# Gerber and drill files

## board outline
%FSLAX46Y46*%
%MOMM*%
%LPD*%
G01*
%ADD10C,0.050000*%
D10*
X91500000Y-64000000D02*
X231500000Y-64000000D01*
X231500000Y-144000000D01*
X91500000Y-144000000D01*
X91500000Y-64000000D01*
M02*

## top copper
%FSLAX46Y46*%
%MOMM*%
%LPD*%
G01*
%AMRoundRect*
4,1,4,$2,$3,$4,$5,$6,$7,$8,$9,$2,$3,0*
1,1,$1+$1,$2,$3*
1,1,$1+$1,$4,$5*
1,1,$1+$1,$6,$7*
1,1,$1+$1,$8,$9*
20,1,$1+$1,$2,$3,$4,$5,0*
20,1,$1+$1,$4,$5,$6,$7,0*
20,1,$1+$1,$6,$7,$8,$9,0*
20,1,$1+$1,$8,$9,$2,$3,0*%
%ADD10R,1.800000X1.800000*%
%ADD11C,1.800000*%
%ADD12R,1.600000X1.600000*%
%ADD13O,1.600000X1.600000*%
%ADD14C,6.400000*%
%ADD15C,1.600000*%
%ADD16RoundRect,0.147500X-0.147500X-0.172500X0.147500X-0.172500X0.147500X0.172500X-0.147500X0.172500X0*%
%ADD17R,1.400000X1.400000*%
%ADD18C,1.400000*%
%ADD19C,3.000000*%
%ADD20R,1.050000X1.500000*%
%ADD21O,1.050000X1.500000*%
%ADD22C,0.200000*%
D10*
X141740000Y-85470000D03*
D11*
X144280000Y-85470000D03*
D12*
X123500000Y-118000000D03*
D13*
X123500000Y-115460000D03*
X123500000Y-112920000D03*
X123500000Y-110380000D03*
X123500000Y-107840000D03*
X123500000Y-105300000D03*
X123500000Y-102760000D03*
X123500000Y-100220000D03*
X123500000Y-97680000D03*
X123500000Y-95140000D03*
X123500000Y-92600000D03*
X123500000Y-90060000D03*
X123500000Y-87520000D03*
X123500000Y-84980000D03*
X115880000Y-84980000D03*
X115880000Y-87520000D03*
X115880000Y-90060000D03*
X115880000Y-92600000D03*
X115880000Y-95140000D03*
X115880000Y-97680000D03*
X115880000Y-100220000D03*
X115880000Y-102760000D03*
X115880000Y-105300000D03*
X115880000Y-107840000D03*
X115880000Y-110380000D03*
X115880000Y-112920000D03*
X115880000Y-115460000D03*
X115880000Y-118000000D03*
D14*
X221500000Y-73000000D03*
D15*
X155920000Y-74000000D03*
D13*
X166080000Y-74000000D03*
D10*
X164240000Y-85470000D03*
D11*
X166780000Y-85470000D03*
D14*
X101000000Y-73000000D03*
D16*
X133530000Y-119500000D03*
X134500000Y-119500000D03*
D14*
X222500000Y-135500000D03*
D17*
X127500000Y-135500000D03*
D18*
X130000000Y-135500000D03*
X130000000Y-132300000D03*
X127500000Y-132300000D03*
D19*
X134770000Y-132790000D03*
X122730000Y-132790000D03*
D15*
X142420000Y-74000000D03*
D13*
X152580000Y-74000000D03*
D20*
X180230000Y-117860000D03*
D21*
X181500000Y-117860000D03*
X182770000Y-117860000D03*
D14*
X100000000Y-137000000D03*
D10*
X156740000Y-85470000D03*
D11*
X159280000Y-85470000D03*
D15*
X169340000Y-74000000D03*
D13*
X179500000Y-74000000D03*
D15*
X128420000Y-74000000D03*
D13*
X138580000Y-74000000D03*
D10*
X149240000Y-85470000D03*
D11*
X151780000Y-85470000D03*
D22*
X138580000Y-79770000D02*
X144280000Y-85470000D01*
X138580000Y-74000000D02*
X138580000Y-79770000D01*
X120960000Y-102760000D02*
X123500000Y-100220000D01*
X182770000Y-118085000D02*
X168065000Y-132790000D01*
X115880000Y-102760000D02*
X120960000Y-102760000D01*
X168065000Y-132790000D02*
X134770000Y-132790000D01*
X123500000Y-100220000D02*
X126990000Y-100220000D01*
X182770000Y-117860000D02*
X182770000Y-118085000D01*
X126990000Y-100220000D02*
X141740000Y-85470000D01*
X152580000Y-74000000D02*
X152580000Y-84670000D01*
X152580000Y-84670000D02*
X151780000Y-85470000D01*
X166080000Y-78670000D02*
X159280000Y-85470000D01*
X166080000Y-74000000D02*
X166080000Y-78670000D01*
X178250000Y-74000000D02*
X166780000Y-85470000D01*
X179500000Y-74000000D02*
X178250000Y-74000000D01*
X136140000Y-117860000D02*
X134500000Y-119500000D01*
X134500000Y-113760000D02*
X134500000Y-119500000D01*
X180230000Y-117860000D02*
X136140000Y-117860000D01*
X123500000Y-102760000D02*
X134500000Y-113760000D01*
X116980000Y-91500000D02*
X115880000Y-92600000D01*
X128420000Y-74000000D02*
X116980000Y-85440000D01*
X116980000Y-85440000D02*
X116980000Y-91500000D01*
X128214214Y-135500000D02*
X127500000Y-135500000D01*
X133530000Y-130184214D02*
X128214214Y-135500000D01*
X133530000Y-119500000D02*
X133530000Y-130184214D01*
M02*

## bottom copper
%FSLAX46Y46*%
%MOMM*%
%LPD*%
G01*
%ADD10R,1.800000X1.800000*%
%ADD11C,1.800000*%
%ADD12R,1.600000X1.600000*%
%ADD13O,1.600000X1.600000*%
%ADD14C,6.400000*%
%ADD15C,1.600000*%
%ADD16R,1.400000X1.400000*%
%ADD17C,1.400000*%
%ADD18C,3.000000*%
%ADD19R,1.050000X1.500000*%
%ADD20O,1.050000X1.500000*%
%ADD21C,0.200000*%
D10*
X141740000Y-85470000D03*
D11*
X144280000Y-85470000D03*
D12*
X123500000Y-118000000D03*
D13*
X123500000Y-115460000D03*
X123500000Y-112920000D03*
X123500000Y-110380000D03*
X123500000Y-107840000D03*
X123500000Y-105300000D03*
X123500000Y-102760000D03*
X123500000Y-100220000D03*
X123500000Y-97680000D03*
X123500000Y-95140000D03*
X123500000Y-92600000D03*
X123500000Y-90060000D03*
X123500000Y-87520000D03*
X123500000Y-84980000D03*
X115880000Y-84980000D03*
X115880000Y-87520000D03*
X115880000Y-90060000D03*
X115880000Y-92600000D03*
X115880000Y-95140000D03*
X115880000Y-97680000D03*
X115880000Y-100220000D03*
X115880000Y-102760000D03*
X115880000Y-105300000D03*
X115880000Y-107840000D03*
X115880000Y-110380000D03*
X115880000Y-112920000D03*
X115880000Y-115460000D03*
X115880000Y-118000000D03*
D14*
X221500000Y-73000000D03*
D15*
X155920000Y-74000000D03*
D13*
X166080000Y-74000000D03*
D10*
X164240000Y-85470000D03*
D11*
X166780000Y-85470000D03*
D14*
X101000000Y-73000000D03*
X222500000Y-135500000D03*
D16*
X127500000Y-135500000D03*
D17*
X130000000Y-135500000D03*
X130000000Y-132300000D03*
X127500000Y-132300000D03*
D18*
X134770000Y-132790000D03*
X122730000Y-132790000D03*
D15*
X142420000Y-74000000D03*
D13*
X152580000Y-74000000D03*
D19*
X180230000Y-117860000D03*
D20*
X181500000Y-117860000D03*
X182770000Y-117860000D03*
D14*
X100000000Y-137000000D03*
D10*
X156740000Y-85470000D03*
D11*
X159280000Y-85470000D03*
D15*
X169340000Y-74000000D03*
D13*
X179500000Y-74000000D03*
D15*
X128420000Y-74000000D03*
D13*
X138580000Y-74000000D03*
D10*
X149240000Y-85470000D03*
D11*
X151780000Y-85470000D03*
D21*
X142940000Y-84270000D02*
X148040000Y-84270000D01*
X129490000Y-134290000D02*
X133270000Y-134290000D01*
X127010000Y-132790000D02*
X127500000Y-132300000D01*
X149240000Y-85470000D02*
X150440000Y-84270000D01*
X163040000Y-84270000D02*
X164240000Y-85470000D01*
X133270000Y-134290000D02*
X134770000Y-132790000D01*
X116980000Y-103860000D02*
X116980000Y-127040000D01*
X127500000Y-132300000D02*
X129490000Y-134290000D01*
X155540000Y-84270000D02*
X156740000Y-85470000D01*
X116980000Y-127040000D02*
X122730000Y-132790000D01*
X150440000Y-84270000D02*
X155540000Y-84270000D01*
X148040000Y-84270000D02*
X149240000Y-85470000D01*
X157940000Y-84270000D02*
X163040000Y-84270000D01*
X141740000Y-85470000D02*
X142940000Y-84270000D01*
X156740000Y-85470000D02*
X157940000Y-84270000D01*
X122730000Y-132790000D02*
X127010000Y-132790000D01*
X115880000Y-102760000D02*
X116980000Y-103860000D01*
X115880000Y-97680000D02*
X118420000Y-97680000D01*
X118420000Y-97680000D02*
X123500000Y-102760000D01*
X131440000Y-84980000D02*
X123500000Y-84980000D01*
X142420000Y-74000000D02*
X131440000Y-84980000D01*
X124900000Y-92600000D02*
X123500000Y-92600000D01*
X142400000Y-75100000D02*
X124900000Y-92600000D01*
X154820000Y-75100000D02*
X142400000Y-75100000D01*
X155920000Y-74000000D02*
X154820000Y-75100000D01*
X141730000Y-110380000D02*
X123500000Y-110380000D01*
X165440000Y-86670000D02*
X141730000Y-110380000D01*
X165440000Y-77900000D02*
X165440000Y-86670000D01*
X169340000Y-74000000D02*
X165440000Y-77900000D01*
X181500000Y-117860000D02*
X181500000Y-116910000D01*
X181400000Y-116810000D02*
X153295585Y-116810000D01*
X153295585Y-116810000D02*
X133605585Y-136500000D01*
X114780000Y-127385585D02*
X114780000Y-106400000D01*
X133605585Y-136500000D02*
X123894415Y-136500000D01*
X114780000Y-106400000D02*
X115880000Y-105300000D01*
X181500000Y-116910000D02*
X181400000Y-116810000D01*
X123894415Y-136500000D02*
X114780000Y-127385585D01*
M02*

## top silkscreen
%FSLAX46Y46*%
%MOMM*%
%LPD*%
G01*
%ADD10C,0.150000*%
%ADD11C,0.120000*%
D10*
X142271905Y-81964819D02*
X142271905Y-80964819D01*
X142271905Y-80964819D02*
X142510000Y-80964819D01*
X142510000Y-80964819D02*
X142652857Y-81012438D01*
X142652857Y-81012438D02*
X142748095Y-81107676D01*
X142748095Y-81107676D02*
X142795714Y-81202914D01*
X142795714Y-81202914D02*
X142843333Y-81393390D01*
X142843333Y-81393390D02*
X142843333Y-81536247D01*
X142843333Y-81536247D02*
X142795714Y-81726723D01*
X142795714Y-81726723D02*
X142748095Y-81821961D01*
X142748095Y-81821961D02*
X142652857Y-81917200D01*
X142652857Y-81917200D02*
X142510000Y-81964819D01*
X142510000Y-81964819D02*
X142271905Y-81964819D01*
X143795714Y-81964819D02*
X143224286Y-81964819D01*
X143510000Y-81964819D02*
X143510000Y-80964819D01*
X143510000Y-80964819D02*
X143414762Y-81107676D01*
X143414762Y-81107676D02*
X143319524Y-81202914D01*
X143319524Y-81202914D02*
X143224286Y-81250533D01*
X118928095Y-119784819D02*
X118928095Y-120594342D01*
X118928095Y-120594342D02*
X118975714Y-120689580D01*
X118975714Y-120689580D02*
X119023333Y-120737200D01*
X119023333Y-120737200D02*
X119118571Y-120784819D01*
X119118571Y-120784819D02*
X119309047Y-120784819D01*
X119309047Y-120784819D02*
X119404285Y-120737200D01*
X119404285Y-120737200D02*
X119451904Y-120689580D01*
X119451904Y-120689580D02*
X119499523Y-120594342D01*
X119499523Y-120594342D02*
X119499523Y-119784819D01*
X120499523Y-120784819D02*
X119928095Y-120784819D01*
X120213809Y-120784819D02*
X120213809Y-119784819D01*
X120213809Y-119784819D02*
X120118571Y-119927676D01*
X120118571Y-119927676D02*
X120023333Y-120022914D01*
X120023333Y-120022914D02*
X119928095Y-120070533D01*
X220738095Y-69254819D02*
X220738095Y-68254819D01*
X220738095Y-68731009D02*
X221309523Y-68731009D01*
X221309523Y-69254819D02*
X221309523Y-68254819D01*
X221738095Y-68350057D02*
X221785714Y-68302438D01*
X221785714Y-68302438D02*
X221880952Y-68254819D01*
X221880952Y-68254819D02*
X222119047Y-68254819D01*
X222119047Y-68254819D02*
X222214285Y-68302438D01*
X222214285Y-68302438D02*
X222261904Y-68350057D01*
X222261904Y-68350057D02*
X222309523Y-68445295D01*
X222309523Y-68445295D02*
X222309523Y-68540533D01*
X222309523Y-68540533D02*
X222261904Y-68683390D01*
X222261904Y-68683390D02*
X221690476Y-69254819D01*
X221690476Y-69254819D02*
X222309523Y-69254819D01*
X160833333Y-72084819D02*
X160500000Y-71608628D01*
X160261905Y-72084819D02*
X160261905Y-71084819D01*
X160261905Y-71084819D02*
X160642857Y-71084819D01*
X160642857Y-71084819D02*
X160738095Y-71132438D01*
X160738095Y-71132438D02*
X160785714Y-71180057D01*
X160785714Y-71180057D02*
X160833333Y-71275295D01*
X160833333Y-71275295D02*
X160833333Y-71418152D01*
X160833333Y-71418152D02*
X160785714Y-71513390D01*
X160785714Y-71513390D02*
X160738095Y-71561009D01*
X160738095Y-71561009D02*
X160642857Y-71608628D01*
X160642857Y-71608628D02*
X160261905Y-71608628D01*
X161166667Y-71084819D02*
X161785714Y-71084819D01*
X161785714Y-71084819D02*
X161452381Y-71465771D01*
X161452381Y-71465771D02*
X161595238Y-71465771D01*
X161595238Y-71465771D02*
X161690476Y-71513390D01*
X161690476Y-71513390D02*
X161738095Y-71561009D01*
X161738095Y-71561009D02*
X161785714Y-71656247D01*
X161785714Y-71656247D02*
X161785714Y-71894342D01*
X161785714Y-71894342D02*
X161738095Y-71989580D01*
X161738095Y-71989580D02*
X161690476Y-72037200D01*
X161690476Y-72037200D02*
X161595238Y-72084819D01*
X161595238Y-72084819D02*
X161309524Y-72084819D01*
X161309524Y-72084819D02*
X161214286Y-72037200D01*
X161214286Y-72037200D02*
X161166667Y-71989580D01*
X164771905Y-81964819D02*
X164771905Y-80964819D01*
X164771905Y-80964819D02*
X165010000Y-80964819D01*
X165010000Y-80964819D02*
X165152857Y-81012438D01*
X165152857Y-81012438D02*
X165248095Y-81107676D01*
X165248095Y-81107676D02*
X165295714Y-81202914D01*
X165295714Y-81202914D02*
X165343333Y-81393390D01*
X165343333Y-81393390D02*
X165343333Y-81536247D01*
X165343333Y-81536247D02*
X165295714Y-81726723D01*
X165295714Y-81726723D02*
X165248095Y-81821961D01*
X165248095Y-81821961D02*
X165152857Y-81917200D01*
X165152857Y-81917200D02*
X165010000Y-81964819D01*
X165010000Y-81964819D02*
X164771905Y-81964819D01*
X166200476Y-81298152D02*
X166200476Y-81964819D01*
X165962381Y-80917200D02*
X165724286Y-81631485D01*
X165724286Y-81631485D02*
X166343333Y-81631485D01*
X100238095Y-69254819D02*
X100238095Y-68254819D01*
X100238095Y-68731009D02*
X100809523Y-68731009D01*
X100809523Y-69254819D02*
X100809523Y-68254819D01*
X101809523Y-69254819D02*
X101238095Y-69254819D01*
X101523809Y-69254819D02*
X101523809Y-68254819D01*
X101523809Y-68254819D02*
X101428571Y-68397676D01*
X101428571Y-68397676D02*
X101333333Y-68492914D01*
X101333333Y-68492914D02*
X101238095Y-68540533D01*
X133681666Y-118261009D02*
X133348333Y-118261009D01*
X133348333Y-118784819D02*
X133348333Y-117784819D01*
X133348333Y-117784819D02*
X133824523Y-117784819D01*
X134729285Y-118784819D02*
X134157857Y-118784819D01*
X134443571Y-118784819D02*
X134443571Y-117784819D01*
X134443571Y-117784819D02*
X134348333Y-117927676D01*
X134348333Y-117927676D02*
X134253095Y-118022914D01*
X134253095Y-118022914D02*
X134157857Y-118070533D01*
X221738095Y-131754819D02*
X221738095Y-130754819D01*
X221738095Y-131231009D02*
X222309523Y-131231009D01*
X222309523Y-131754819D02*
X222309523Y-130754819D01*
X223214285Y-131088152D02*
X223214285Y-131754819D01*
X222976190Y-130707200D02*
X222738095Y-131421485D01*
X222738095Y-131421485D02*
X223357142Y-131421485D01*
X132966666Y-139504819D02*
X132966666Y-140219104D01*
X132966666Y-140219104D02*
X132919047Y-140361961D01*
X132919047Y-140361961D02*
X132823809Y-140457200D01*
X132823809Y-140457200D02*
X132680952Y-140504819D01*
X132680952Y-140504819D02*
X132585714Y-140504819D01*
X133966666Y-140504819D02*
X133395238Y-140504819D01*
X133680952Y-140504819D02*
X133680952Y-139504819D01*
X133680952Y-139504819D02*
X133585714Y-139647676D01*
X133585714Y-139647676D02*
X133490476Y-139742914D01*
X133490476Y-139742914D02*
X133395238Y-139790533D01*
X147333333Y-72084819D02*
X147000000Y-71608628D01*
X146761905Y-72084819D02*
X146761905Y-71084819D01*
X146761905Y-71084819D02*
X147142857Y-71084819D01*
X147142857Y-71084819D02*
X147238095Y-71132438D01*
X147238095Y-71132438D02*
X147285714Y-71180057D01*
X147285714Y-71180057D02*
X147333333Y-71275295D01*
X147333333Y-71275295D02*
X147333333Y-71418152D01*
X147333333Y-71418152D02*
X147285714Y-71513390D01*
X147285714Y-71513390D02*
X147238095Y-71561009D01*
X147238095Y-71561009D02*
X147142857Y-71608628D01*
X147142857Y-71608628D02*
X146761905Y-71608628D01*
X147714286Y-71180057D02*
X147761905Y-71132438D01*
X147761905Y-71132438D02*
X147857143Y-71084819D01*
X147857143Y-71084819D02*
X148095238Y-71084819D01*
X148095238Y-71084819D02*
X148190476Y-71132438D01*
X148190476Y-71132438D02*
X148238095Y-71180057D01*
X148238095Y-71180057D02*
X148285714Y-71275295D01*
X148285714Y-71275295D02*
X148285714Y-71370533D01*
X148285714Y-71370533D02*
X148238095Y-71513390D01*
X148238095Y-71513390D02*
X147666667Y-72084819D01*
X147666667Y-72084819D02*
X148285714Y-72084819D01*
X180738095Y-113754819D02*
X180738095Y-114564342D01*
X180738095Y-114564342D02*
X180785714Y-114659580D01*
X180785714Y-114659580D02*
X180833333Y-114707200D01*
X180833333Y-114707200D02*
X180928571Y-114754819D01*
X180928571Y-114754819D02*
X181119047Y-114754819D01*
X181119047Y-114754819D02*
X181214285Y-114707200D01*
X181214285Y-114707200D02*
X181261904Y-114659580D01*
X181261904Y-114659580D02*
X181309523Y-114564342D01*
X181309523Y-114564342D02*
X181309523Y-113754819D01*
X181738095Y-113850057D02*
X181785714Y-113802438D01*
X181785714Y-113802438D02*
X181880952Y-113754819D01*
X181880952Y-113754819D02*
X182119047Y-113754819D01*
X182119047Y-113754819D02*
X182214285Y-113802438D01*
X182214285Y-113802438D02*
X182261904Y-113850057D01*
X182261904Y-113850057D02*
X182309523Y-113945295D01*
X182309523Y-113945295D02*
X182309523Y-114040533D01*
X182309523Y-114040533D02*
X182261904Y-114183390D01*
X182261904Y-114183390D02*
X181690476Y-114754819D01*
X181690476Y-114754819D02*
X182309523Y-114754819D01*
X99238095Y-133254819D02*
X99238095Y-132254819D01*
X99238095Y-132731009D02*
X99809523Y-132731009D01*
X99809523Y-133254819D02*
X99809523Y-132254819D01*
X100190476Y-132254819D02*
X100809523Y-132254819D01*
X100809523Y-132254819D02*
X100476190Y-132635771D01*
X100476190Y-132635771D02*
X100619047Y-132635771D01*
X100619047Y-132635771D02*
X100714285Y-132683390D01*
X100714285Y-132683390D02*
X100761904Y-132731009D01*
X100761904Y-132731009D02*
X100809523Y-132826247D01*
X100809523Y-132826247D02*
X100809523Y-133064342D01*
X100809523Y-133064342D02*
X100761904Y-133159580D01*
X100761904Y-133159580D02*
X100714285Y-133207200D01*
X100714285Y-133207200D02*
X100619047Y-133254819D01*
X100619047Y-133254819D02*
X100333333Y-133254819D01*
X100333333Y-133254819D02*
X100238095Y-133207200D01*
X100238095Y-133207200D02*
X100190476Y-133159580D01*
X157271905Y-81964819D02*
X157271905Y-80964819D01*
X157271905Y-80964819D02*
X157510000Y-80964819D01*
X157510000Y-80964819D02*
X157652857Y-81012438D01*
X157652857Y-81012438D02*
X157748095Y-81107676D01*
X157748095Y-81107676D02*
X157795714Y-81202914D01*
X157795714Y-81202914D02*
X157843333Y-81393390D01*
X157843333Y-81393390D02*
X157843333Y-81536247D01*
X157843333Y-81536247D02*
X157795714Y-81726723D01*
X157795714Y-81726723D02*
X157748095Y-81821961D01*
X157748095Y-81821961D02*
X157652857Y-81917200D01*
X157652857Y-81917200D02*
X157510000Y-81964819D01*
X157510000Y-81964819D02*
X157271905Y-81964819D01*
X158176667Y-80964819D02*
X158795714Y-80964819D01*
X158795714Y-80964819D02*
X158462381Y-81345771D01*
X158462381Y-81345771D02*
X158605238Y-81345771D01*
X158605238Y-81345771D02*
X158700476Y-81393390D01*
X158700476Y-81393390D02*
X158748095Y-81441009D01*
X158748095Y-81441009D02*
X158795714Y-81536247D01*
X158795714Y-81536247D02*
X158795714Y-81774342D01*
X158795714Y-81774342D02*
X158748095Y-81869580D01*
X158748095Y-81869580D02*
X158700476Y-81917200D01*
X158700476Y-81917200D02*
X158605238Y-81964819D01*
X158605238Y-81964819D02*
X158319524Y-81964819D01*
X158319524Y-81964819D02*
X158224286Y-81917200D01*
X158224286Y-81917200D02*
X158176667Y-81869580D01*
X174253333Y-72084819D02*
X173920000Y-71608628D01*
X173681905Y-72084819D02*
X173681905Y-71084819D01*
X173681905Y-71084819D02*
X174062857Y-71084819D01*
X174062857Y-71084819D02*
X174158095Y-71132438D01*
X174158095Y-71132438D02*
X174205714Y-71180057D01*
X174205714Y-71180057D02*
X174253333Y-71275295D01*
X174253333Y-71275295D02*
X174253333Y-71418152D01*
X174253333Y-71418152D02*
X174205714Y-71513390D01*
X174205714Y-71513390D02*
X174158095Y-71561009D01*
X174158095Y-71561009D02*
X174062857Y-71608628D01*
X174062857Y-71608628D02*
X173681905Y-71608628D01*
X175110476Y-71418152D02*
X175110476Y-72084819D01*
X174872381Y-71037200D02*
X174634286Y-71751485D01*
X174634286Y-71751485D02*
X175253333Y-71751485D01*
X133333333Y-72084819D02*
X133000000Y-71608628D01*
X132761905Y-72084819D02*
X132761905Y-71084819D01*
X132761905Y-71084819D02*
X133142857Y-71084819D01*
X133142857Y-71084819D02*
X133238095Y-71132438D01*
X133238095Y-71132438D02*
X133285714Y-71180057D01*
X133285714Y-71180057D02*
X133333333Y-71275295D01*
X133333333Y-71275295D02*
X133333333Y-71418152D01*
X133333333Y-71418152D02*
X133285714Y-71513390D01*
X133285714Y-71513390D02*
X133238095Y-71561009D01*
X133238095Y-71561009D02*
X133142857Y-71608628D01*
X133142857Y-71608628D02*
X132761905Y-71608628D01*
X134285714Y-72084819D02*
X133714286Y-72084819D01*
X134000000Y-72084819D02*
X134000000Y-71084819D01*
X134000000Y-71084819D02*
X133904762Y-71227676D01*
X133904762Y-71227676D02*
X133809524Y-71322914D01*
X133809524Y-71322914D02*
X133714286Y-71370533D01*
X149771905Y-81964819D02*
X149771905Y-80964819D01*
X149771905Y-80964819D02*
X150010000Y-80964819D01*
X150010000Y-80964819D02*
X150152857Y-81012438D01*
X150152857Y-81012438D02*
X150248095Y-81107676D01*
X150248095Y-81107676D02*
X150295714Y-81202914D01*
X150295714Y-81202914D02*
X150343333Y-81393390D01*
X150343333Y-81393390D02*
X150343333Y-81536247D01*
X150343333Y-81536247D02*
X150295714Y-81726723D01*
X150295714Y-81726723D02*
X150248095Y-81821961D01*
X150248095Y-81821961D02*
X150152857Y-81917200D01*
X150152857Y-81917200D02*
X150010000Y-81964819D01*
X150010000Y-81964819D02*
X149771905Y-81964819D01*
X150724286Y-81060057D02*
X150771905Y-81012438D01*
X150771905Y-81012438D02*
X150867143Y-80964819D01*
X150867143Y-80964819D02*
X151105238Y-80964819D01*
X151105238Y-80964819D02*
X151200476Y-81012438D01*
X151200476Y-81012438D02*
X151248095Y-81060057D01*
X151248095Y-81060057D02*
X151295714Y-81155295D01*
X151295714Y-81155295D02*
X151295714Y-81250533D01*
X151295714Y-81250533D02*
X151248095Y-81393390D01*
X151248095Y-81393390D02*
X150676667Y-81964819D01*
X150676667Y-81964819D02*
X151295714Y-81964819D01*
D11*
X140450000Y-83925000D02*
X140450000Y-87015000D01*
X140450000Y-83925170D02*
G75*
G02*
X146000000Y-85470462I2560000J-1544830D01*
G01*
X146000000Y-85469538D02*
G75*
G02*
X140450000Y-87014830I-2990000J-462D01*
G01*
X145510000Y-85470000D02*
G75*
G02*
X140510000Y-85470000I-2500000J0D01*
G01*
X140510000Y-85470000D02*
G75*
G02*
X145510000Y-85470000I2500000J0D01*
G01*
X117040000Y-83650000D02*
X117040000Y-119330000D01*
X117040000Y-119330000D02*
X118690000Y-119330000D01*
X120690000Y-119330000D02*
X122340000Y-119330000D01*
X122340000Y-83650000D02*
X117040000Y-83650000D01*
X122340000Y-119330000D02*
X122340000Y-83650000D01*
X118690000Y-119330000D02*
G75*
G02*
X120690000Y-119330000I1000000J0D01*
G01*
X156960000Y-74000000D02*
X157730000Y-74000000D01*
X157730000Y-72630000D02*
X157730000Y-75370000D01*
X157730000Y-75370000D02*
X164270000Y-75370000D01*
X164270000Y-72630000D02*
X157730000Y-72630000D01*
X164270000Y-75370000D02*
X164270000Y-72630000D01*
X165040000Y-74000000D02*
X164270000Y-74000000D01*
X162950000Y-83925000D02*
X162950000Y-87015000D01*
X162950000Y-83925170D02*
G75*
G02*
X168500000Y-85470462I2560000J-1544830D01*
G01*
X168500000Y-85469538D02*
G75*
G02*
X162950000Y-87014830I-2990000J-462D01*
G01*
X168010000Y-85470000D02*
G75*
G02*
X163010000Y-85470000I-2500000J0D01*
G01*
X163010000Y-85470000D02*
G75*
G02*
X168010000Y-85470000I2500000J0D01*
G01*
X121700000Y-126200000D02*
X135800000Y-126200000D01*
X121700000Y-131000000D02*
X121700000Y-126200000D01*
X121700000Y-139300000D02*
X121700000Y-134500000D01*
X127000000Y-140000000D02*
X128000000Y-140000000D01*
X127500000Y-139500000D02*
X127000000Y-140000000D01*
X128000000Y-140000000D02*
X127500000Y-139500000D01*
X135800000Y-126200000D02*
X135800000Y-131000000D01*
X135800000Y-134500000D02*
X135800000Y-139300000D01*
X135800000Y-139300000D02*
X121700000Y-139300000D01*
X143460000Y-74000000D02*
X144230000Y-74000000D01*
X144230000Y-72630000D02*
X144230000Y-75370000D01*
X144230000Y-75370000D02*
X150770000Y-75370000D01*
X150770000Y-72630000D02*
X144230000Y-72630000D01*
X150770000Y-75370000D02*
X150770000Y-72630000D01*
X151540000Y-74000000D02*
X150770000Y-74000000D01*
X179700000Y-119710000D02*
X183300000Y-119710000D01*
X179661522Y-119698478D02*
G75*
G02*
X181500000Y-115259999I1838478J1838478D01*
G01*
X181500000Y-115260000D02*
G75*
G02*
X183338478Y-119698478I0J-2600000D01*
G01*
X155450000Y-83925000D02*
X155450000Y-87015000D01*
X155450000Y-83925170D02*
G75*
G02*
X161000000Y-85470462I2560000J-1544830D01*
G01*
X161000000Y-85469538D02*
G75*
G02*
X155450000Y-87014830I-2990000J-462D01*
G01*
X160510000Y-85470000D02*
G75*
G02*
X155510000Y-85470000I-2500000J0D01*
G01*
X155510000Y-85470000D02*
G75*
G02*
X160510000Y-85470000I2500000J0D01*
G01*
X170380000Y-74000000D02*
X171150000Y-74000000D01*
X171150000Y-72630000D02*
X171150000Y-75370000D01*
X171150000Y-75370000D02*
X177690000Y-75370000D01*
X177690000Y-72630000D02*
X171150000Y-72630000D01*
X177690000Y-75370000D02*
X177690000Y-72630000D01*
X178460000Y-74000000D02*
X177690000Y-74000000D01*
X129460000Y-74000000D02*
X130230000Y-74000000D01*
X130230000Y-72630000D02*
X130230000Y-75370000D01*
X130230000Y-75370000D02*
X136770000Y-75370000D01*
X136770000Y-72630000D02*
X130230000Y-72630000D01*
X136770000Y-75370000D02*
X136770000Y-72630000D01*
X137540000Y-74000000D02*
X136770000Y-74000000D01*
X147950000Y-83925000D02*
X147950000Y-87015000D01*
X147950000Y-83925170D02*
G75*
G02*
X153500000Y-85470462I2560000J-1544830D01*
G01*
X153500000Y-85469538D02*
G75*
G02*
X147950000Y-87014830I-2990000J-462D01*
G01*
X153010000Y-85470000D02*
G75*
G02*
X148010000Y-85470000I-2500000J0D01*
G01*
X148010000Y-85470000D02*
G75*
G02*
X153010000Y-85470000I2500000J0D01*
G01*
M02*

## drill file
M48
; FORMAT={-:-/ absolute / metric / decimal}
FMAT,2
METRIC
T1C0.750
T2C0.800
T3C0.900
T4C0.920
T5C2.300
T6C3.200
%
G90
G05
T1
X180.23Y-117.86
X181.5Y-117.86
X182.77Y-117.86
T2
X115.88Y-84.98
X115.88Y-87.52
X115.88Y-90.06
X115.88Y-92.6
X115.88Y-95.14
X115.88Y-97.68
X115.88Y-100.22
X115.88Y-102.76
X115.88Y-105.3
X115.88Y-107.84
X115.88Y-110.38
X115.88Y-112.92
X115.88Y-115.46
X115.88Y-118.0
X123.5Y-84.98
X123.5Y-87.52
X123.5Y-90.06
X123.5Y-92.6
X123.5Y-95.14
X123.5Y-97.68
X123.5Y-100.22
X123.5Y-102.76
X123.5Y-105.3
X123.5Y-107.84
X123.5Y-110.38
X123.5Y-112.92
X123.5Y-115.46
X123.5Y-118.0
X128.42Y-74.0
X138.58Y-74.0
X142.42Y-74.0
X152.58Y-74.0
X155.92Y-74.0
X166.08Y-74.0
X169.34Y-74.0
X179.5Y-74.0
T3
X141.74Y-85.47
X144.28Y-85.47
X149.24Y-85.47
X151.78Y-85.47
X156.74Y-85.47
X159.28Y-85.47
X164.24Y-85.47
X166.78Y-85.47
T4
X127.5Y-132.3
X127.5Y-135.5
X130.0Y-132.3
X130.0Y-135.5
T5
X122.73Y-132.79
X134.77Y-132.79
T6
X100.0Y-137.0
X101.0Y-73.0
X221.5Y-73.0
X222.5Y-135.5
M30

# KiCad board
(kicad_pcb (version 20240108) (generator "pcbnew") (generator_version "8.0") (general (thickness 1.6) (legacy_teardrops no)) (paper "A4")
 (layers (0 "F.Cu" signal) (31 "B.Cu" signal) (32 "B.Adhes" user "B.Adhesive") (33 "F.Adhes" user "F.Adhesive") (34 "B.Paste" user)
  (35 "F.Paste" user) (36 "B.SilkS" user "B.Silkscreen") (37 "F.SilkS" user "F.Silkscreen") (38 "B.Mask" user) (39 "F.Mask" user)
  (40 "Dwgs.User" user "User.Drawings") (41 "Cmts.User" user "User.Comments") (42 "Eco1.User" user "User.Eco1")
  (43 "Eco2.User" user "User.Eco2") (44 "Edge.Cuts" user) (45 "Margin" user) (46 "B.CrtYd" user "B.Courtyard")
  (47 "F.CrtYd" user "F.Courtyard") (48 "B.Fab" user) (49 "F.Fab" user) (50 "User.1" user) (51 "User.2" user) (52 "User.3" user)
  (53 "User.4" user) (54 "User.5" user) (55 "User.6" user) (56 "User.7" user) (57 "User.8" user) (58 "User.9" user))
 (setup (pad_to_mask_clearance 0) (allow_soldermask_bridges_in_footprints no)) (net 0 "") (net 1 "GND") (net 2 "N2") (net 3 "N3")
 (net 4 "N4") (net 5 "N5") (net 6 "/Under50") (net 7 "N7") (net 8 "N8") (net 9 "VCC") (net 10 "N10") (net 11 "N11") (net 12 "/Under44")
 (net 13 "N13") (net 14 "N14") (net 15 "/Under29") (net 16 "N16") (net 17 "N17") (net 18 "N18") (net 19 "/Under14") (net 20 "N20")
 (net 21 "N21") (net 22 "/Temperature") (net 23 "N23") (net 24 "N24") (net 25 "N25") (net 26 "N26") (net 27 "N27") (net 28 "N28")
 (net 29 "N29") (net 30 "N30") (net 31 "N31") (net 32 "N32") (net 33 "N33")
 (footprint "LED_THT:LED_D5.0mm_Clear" (layer "F.Cu") (at 141.74 85.47)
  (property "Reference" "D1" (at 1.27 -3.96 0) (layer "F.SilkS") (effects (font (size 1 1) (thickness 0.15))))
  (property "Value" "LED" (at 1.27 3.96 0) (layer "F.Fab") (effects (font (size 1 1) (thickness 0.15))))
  (fp_line (start -1.29 -1.545) (end -1.29 1.545) (stroke (width 0.12) (type solid)) (layer "F.SilkS"))
  (fp_arc (start -1.29 -1.54483) (mid 2.072002 -2.880433) (end 4.26 0.000462) (stroke (width 0.12) (type solid)) (layer "F.SilkS"))
  (fp_arc (start 4.26 -0.000462) (mid 2.072002 2.880433) (end -1.29 1.54483) (stroke (width 0.12) (type solid)) (layer "F.SilkS"))
  (fp_circle (center 1.27 0) (end 3.77 0) (stroke (width 0.12) (type solid)) (fill none) (layer "F.SilkS"))
  (pad "1" thru_hole rect (at 0 0) (size 1.8 1.8) (drill 0.9) (layers "*.Cu" "*.Mask") (remove_unused_layers no) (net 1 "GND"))
  (pad "2" thru_hole circle (at 2.54 0) (size 1.8 1.8) (drill 0.9) (layers "*.Cu" "*.Mask") (remove_unused_layers no) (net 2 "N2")))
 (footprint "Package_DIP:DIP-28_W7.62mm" (layer "F.Cu") (at 123.5 118 180)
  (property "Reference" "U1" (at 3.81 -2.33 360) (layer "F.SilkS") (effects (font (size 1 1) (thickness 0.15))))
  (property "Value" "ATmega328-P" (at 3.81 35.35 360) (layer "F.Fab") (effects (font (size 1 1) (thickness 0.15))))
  (fp_line (start 6.46 34.35) (end 6.46 -1.33) (stroke (width 0.12) (type solid)) (layer "F.SilkS"))
  (fp_line (start 6.46 -1.33) (end 4.81 -1.33) (stroke (width 0.12) (type solid)) (layer "F.SilkS"))
  (fp_line (start 2.81 -1.33) (end 1.16 -1.33) (stroke (width 0.12) (type solid)) (layer "F.SilkS"))
  (fp_line (start 1.16 34.35) (end 6.46 34.35) (stroke (width 0.12) (type solid)) (layer "F.SilkS"))
  (fp_line (start 1.16 -1.33) (end 1.16 34.35) (stroke (width 0.12) (type solid)) (layer "F.SilkS"))
  (fp_arc (start 4.81 -1.33) (mid 3.81 -0.33) (end 2.81 -1.33) (stroke (width 0.12) (type solid)) (layer "F.SilkS"))
  (pad "1" thru_hole rect (at 0 0 180) (size 1.6 1.6) (drill 0.8) (layers "*.Cu" "*.Mask") (remove_unused_layers no) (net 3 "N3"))
  (pad "2" thru_hole oval (at 0 2.54 180) (size 1.6 1.6) (drill 0.8) (layers "*.Cu" "*.Mask") (remove_unused_layers no) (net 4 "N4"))
  (pad "3" thru_hole oval (at 0 5.08 180) (size 1.6 1.6) (drill 0.8) (layers "*.Cu" "*.Mask") (remove_unused_layers no) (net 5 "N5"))
  (pad "4" thru_hole oval (at 0 7.62 180) (size 1.6 1.6) (drill 0.8) (layers "*.Cu" "*.Mask") (remove_unused_layers no) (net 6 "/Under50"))
  (pad "5" thru_hole oval (at 0 10.16 180) (size 1.6 1.6) (drill 0.8) (layers "*.Cu" "*.Mask") (remove_unused_layers no) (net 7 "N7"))
  (pad "6" thru_hole oval (at 0 12.7 180) (size 1.6 1.6) (drill 0.8) (layers "*.Cu" "*.Mask") (remove_unused_layers no) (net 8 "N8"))
  (pad "7" thru_hole oval (at 0 15.24 180) (size 1.6 1.6) (drill 0.8) (layers "*.Cu" "*.Mask") (remove_unused_layers no) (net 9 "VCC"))
  (pad "8" thru_hole oval (at 0 17.78 180) (size 1.6 1.6) (drill 0.8) (layers "*.Cu" "*.Mask") (remove_unused_layers no) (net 1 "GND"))
  (pad "9" thru_hole oval (at 0 20.32 180) (size 1.6 1.6) (drill 0.8) (layers "*.Cu" "*.Mask") (remove_unused_layers no) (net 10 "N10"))
  (pad "10" thru_hole oval (at 0 22.86 180) (size 1.6 1.6) (drill 0.8) (layers "*.Cu" "*.Mask") (remove_unused_layers no) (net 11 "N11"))
  (pad "11" thru_hole oval (at 0 25.4 180) (size 1.6 1.6) (drill 0.8) (layers "*.Cu" "*.Mask") (remove_unused_layers no) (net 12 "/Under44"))
  (pad "12" thru_hole oval (at 0 27.94 180) (size 1.6 1.6) (drill 0.8) (layers "*.Cu" "*.Mask") (remove_unused_layers no) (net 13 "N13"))
  (pad "13" thru_hole oval (at 0 30.48 180) (size 1.6 1.6) (drill 0.8) (layers "*.Cu" "*.Mask") (remove_unused_layers no) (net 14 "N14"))
  (pad "14" thru_hole oval (at 0 33.02 180) (size 1.6 1.6) (drill 0.8) (layers "*.Cu" "*.Mask") (remove_unused_layers no)
   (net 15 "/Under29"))
  (pad "15" thru_hole oval (at 7.62 33.02 180) (size 1.6 1.6) (drill 0.8) (layers "*.Cu" "*.Mask") (remove_unused_layers no) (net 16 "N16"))
  (pad "16" thru_hole oval (at 7.62 30.48 180) (size 1.6 1.6) (drill 0.8) (layers "*.Cu" "*.Mask") (remove_unused_layers no) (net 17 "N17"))
  (pad "17" thru_hole oval (at 7.62 27.94 180) (size 1.6 1.6) (drill 0.8) (layers "*.Cu" "*.Mask") (remove_unused_layers no) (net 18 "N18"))
  (pad "18" thru_hole oval (at 7.62 25.4 180) (size 1.6 1.6) (drill 0.8) (layers "*.Cu" "*.Mask") (remove_unused_layers no)
   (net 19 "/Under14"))
  (pad "19" thru_hole oval (at 7.62 22.86 180) (size 1.6 1.6) (drill 0.8) (layers "*.Cu" "*.Mask") (remove_unused_layers no) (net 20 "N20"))
  (pad "20" thru_hole oval (at 7.62 20.32 180) (size 1.6 1.6) (drill 0.8) (layers "*.Cu" "*.Mask") (remove_unused_layers no) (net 9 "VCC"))
  (pad "21" thru_hole oval (at 7.62 17.78 180) (size 1.6 1.6) (drill 0.8) (layers "*.Cu" "*.Mask") (remove_unused_layers no) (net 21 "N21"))
  (pad "22" thru_hole oval (at 7.62 15.24 180) (size 1.6 1.6) (drill 0.8) (layers "*.Cu" "*.Mask") (remove_unused_layers no) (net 1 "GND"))
  (pad "23" thru_hole oval (at 7.62 12.7 180) (size 1.6 1.6) (drill 0.8) (layers "*.Cu" "*.Mask") (remove_unused_layers no)
   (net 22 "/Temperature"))
  (pad "24" thru_hole oval (at 7.62 10.16 180) (size 1.6 1.6) (drill 0.8) (layers "*.Cu" "*.Mask") (remove_unused_layers no) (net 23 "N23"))
  (pad "25" thru_hole oval (at 7.62 7.62 180) (size 1.6 1.6) (drill 0.8) (layers "*.Cu" "*.Mask") (remove_unused_layers no) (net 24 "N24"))
  (pad "26" thru_hole oval (at 7.62 5.08 180) (size 1.6 1.6) (drill 0.8) (layers "*.Cu" "*.Mask") (remove_unused_layers no) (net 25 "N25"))
  (pad "27" thru_hole oval (at 7.62 2.54 180) (size 1.6 1.6) (drill 0.8) (layers "*.Cu" "*.Mask") (remove_unused_layers no) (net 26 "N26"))
  (pad "28" thru_hole oval (at 7.62 0 180) (size 1.6 1.6) (drill 0.8) (layers "*.Cu" "*.Mask") (remove_unused_layers no) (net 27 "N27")))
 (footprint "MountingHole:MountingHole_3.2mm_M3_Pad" (layer "F.Cu") (at 221.5 73)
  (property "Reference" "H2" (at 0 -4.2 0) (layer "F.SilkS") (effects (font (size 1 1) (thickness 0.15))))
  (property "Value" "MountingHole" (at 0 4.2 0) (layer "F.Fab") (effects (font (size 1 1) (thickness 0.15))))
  (pad "1" thru_hole circle (at 0 0) (size 6.4 6.4) (drill 3.2) (layers "*.Cu" "*.Mask") (remove_unused_layers no)))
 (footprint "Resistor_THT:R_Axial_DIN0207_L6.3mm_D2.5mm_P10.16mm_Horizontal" (layer "F.Cu") (at 155.92 74)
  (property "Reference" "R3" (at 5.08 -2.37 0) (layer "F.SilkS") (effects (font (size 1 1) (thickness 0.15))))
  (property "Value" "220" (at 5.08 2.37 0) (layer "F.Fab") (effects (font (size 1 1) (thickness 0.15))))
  (fp_line (start 1.04 0) (end 1.81 0) (stroke (width 0.12) (type solid)) (layer "F.SilkS"))
  (fp_line (start 1.81 -1.37) (end 1.81 1.37) (stroke (width 0.12) (type solid)) (layer "F.SilkS"))
  (fp_line (start 1.81 1.37) (end 8.35 1.37) (stroke (width 0.12) (type solid)) (layer "F.SilkS"))
  (fp_line (start 8.35 -1.37) (end 1.81 -1.37) (stroke (width 0.12) (type solid)) (layer "F.SilkS"))
  (fp_line (start 8.35 1.37) (end 8.35 -1.37) (stroke (width 0.12) (type solid)) (layer "F.SilkS"))
  (fp_line (start 9.12 0) (end 8.35 0) (stroke (width 0.12) (type solid)) (layer "F.SilkS"))
  (pad "1" thru_hole circle (at 0 0) (size 1.6 1.6) (drill 0.8) (layers "*.Cu" "*.Mask") (remove_unused_layers no) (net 12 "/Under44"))
  (pad "2" thru_hole oval (at 10.16 0) (size 1.6 1.6) (drill 0.8) (layers "*.Cu" "*.Mask") (remove_unused_layers no) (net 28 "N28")))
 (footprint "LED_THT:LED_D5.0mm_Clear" (layer "F.Cu") (at 164.24 85.47)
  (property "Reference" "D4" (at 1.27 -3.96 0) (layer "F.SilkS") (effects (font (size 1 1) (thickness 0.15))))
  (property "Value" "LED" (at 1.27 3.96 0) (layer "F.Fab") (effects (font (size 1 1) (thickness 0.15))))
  (fp_line (start -1.29 -1.545) (end -1.29 1.545) (stroke (width 0.12) (type solid)) (layer "F.SilkS"))
  (fp_arc (start -1.29 -1.54483) (mid 2.072002 -2.880433) (end 4.26 0.000462) (stroke (width 0.12) (type solid)) (layer "F.SilkS"))
  (fp_arc (start 4.26 -0.000462) (mid 2.072002 2.880433) (end -1.29 1.54483) (stroke (width 0.12) (type solid)) (layer "F.SilkS"))
  (fp_circle (center 1.27 0) (end 3.77 0) (stroke (width 0.12) (type solid)) (fill none) (layer "F.SilkS"))
  (pad "1" thru_hole rect (at 0 0) (size 1.8 1.8) (drill 0.9) (layers "*.Cu" "*.Mask") (remove_unused_layers no) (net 1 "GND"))
  (pad "2" thru_hole circle (at 2.54 0) (size 1.8 1.8) (drill 0.9) (layers "*.Cu" "*.Mask") (remove_unused_layers no) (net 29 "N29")))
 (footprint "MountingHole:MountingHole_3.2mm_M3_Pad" (layer "F.Cu") (at 101 73)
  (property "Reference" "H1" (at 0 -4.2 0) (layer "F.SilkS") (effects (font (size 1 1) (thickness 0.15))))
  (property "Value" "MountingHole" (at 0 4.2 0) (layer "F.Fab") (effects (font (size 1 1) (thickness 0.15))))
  (pad "1" thru_hole circle (at 0 0) (size 6.4 6.4) (drill 3.2) (layers "*.Cu" "*.Mask") (remove_unused_layers no)))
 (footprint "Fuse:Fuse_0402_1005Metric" (layer "F.Cu") (at 134.015 119.5)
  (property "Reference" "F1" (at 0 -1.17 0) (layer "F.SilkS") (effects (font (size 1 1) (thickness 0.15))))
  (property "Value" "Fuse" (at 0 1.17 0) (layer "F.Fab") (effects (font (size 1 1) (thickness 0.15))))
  (pad "1" smd roundrect (at -0.485 0) (size 0.59 0.64) (layers "F.Cu" "F.Paste" "F.Mask") (roundrect_rratio 0.25) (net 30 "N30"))
  (pad "2" smd roundrect (at 0.485 0) (size 0.59 0.64) (layers "F.Cu" "F.Paste" "F.Mask") (roundrect_rratio 0.25) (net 9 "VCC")))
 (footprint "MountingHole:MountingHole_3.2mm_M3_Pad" (layer "F.Cu") (at 222.5 135.5)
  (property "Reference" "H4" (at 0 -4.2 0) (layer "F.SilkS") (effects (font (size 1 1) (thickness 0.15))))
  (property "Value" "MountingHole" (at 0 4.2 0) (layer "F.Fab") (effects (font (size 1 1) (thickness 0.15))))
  (pad "1" thru_hole circle (at 0 0) (size 6.4 6.4) (drill 3.2) (layers "*.Cu" "*.Mask") (remove_unused_layers no)))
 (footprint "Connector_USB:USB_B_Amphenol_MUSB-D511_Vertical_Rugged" (layer "F.Cu") (at 127.5 135.5 180)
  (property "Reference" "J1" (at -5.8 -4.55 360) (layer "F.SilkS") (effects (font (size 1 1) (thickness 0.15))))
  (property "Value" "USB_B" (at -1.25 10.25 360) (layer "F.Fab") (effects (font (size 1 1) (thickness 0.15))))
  (fp_line (start 5.8 9.3) (end -8.3 9.3) (stroke (width 0.12) (type solid)) (layer "F.SilkS"))
  (fp_line (start 5.8 4.5) (end 5.8 9.3) (stroke (width 0.12) (type solid)) (layer "F.SilkS"))
  (fp_line (start 5.8 -3.8) (end 5.8 1) (stroke (width 0.12) (type solid)) (layer "F.SilkS"))
  (fp_line (start 0.5 -4.5) (end -0.5 -4.5) (stroke (width 0.12) (type solid)) (layer "F.SilkS"))
  (fp_line (start 0 -4) (end 0.5 -4.5) (stroke (width 0.12) (type solid)) (layer "F.SilkS"))
  (fp_line (start -0.5 -4.5) (end 0 -4) (stroke (width 0.12) (type solid)) (layer "F.SilkS"))
  (fp_line (start -8.3 9.3) (end -8.3 4.5) (stroke (width 0.12) (type solid)) (layer "F.SilkS"))
  (fp_line (start -8.3 1) (end -8.3 -3.8) (stroke (width 0.12) (type solid)) (layer "F.SilkS"))
  (fp_line (start -8.3 -3.8) (end 5.8 -3.8) (stroke (width 0.12) (type solid)) (layer "F.SilkS"))
  (pad "1" thru_hole rect (at 0 0 180) (size 1.4 1.4) (drill 0.92) (layers "*.Cu" "*.Mask") (remove_unused_layers no) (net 30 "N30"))
  (pad "2" thru_hole circle (at -2.5 0 180) (size 1.4 1.4) (drill 0.92) (layers "*.Cu" "*.Mask") (remove_unused_layers no) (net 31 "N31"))
  (pad "3" thru_hole circle (at -2.5 3.2 180) (size 1.4 1.4) (drill 0.92) (layers "*.Cu" "*.Mask") (remove_unused_layers no) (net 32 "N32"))
  (pad "4" thru_hole circle (at 0 3.2 180) (size 1.4 1.4) (drill 0.92) (layers "*.Cu" "*.Mask") (remove_unused_layers no) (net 1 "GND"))
  (pad "5" thru_hole circle (at -7.27 2.71 180) (size 3 3) (drill 2.3) (layers "*.Cu" "*.Mask") (remove_unused_layers no) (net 1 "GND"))
  (pad "5" thru_hole circle (at 4.77 2.71 180) (size 3 3) (drill 2.3) (layers "*.Cu" "*.Mask") (remove_unused_layers no) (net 1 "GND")))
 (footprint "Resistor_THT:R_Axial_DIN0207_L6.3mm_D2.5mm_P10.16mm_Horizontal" (layer "F.Cu") (at 142.42 74)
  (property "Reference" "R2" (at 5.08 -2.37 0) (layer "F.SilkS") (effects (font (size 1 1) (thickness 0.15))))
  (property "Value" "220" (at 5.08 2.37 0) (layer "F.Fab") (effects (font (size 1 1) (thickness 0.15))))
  (fp_line (start 1.04 0) (end 1.81 0) (stroke (width 0.12) (type solid)) (layer "F.SilkS"))
  (fp_line (start 1.81 -1.37) (end 1.81 1.37) (stroke (width 0.12) (type solid)) (layer "F.SilkS"))
  (fp_line (start 1.81 1.37) (end 8.35 1.37) (stroke (width 0.12) (type solid)) (layer "F.SilkS"))
  (fp_line (start 8.35 -1.37) (end 1.81 -1.37) (stroke (width 0.12) (type solid)) (layer "F.SilkS"))
  (fp_line (start 8.35 1.37) (end 8.35 -1.37) (stroke (width 0.12) (type solid)) (layer "F.SilkS"))
  (fp_line (start 9.12 0) (end 8.35 0) (stroke (width 0.12) (type solid)) (layer "F.SilkS"))
  (pad "1" thru_hole circle (at 0 0) (size 1.6 1.6) (drill 0.8) (layers "*.Cu" "*.Mask") (remove_unused_layers no) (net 15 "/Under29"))
  (pad "2" thru_hole oval (at 10.16 0) (size 1.6 1.6) (drill 0.8) (layers "*.Cu" "*.Mask") (remove_unused_layers no) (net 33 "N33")))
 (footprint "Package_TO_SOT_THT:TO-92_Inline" (layer "F.Cu") (at 180.23 117.86)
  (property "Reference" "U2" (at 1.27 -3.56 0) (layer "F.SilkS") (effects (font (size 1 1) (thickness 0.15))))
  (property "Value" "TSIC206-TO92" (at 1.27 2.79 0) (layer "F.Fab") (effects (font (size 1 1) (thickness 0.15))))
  (fp_line (start -0.53 1.85) (end 3.07 1.85) (stroke (width 0.12) (type solid)) (layer "F.SilkS"))
  (fp_arc (start -0.568478 1.838478) (mid -1.132087 -0.994977) (end 1.27 -2.6) (stroke (width 0.12) (type solid)) (layer "F.SilkS"))
  (fp_arc (start 1.27 -2.6) (mid 3.672087 -0.994977) (end 3.108478 1.838478) (stroke (width 0.12) (type solid)) (layer "F.SilkS"))
  (pad "1" thru_hole rect (at 0 0) (size 1.05 1.5) (drill 0.75) (layers "*.Cu" "*.Mask") (remove_unused_layers no) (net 9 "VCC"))
  (pad "2" thru_hole oval (at 1.27 0) (size 1.05 1.5) (drill 0.75) (layers "*.Cu" "*.Mask") (remove_unused_layers no)
   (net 22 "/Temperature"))
  (pad "3" thru_hole oval (at 2.54 0) (size 1.05 1.5) (drill 0.75) (layers "*.Cu" "*.Mask") (remove_unused_layers no) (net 1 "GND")))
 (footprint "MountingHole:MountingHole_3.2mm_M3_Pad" (layer "F.Cu") (at 100 137)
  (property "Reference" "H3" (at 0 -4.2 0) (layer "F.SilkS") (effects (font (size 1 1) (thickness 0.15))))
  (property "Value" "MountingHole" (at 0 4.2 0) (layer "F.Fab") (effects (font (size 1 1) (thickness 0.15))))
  (pad "1" thru_hole circle (at 0 0) (size 6.4 6.4) (drill 3.2) (layers "*.Cu" "*.Mask") (remove_unused_layers no)))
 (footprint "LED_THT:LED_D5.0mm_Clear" (layer "F.Cu") (at 156.74 85.47)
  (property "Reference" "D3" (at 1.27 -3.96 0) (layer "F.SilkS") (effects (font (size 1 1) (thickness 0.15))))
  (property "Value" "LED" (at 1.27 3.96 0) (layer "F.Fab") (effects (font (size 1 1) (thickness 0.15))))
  (fp_line (start -1.29 -1.545) (end -1.29 1.545) (stroke (width 0.12) (type solid)) (layer "F.SilkS"))
  (fp_arc (start -1.29 -1.54483) (mid 2.072002 -2.880433) (end 4.26 0.000462) (stroke (width 0.12) (type solid)) (layer "F.SilkS"))
  (fp_arc (start 4.26 -0.000462) (mid 2.072002 2.880433) (end -1.29 1.54483) (stroke (width 0.12) (type solid)) (layer "F.SilkS"))
  (fp_circle (center 1.27 0) (end 3.77 0) (stroke (width 0.12) (type solid)) (fill none) (layer "F.SilkS"))
  (pad "1" thru_hole rect (at 0 0) (size 1.8 1.8) (drill 0.9) (layers "*.Cu" "*.Mask") (remove_unused_layers no) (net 1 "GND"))
  (pad "2" thru_hole circle (at 2.54 0) (size 1.8 1.8) (drill 0.9) (layers "*.Cu" "*.Mask") (remove_unused_layers no) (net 28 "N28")))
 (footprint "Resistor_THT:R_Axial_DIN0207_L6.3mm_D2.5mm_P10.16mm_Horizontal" (layer "F.Cu") (at 169.34 74)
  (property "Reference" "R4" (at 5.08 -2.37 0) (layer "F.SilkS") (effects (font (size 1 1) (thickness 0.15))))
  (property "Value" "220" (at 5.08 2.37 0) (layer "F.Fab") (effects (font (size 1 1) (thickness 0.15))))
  (fp_line (start 1.04 0) (end 1.81 0) (stroke (width 0.12) (type solid)) (layer "F.SilkS"))
  (fp_line (start 1.81 -1.37) (end 1.81 1.37) (stroke (width 0.12) (type solid)) (layer "F.SilkS"))
  (fp_line (start 1.81 1.37) (end 8.35 1.37) (stroke (width 0.12) (type solid)) (layer "F.SilkS"))
  (fp_line (start 8.35 -1.37) (end 1.81 -1.37) (stroke (width 0.12) (type solid)) (layer "F.SilkS"))
  (fp_line (start 8.35 1.37) (end 8.35 -1.37) (stroke (width 0.12) (type solid)) (layer "F.SilkS"))
  (fp_line (start 9.12 0) (end 8.35 0) (stroke (width 0.12) (type solid)) (layer "F.SilkS"))
  (pad "1" thru_hole circle (at 0 0) (size 1.6 1.6) (drill 0.8) (layers "*.Cu" "*.Mask") (remove_unused_layers no) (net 6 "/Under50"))
  (pad "2" thru_hole oval (at 10.16 0) (size 1.6 1.6) (drill 0.8) (layers "*.Cu" "*.Mask") (remove_unused_layers no) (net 29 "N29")))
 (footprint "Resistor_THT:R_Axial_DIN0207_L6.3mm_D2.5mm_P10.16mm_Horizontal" (layer "F.Cu") (at 128.42 74)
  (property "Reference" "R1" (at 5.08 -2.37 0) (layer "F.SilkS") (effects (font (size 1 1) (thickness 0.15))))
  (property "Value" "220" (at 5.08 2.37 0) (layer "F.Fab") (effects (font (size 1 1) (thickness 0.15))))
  (fp_line (start 1.04 0) (end 1.81 0) (stroke (width 0.12) (type solid)) (layer "F.SilkS"))
  (fp_line (start 1.81 -1.37) (end 1.81 1.37) (stroke (width 0.12) (type solid)) (layer "F.SilkS"))
  (fp_line (start 1.81 1.37) (end 8.35 1.37) (stroke (width 0.12) (type solid)) (layer "F.SilkS"))
  (fp_line (start 8.35 -1.37) (end 1.81 -1.37) (stroke (width 0.12) (type solid)) (layer "F.SilkS"))
  (fp_line (start 8.35 1.37) (end 8.35 -1.37) (stroke (width 0.12) (type solid)) (layer "F.SilkS"))
  (fp_line (start 9.12 0) (end 8.35 0) (stroke (width 0.12) (type solid)) (layer "F.SilkS"))
  (pad "1" thru_hole circle (at 0 0) (size 1.6 1.6) (drill 0.8) (layers "*.Cu" "*.Mask") (remove_unused_layers no) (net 19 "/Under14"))
  (pad "2" thru_hole oval (at 10.16 0) (size 1.6 1.6) (drill 0.8) (layers "*.Cu" "*.Mask") (remove_unused_layers no) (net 2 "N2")))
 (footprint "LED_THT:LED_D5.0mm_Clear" (layer "F.Cu") (at 149.24 85.47)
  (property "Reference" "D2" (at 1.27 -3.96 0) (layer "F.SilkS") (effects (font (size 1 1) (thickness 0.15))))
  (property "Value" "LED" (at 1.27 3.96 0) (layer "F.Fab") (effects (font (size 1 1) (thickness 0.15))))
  (fp_line (start -1.29 -1.545) (end -1.29 1.545) (stroke (width 0.12) (type solid)) (layer "F.SilkS"))
  (fp_arc (start -1.29 -1.54483) (mid 2.072002 -2.880433) (end 4.26 0.000462) (stroke (width 0.12) (type solid)) (layer "F.SilkS"))
  (fp_arc (start 4.26 -0.000462) (mid 2.072002 2.880433) (end -1.29 1.54483) (stroke (width 0.12) (type solid)) (layer "F.SilkS"))
  (fp_circle (center 1.27 0) (end 3.77 0) (stroke (width 0.12) (type solid)) (fill none) (layer "F.SilkS"))
  (pad "1" thru_hole rect (at 0 0) (size 1.8 1.8) (drill 0.9) (layers "*.Cu" "*.Mask") (remove_unused_layers no) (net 1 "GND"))
  (pad "2" thru_hole circle (at 2.54 0) (size 1.8 1.8) (drill 0.9) (layers "*.Cu" "*.Mask") (remove_unused_layers no) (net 33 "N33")))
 (gr_rect (start 91.5 64) (end 231.5 144) (stroke (width 0.05) (type default)) (fill none) (layer "Edge.Cuts"))
 (segment (start 138.58 79.77) (end 144.28 85.47) (width 0.2) (layer "F.Cu") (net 2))
 (segment (start 138.58 74) (end 138.58 79.77) (width 0.2) (layer "F.Cu") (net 2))
 (segment (start 120.96 102.76) (end 123.5 100.22) (width 0.2) (layer "F.Cu") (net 1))
 (segment (start 182.77 118.085) (end 168.065 132.79) (width 0.2) (layer "F.Cu") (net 1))
 (segment (start 115.88 102.76) (end 120.96 102.76) (width 0.2) (layer "F.Cu") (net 1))
 (segment (start 168.065 132.79) (end 134.77 132.79) (width 0.2) (layer "F.Cu") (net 1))
 (segment (start 123.5 100.22) (end 126.99 100.22) (width 0.2) (layer "F.Cu") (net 1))
 (segment (start 182.77 117.86) (end 182.77 118.085) (width 0.2) (layer "F.Cu") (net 1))
 (segment (start 126.99 100.22) (end 141.74 85.47) (width 0.2) (layer "F.Cu") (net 1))
 (segment (start 142.94 84.27) (end 148.04 84.27) (width 0.2) (layer "B.Cu") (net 1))
 (segment (start 129.49 134.29) (end 133.27 134.29) (width 0.2) (layer "B.Cu") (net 1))
 (segment (start 127.01 132.79) (end 127.5 132.3) (width 0.2) (layer "B.Cu") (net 1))
 (segment (start 149.24 85.47) (end 150.44 84.27) (width 0.2) (layer "B.Cu") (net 1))
 (segment (start 163.04 84.27) (end 164.24 85.47) (width 0.2) (layer "B.Cu") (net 1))
 (segment (start 133.27 134.29) (end 134.77 132.79) (width 0.2) (layer "B.Cu") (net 1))
 (segment (start 116.98 103.86) (end 116.98 127.04) (width 0.2) (layer "B.Cu") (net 1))
 (segment (start 127.5 132.3) (end 129.49 134.29) (width 0.2) (layer "B.Cu") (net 1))
 (segment (start 155.54 84.27) (end 156.74 85.47) (width 0.2) (layer "B.Cu") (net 1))
 (segment (start 116.98 127.04) (end 122.73 132.79) (width 0.2) (layer "B.Cu") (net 1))
 (segment (start 150.44 84.27) (end 155.54 84.27) (width 0.2) (layer "B.Cu") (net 1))
 (segment (start 148.04 84.27) (end 149.24 85.47) (width 0.2) (layer "B.Cu") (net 1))
 (segment (start 157.94 84.27) (end 163.04 84.27) (width 0.2) (layer "B.Cu") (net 1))
 (segment (start 141.74 85.47) (end 142.94 84.27) (width 0.2) (layer "B.Cu") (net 1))
 (segment (start 156.74 85.47) (end 157.94 84.27) (width 0.2) (layer "B.Cu") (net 1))
 (segment (start 122.73 132.79) (end 127.01 132.79) (width 0.2) (layer "B.Cu") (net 1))
 (segment (start 115.88 102.76) (end 116.98 103.86) (width 0.2) (layer "B.Cu") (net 1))
 (segment (start 152.58 74) (end 152.58 84.67) (width 0.2) (layer "F.Cu") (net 33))
 (segment (start 152.58 84.67) (end 151.78 85.47) (width 0.2) (layer "F.Cu") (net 33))
 (segment (start 166.08 78.67) (end 159.28 85.47) (width 0.2) (layer "F.Cu") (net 28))
 (segment (start 166.08 74) (end 166.08 78.67) (width 0.2) (layer "F.Cu") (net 28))
 (segment (start 178.25 74) (end 166.78 85.47) (width 0.2) (layer "F.Cu") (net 29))
 (segment (start 179.5 74) (end 178.25 74) (width 0.2) (layer "F.Cu") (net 29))
 (segment (start 136.14 117.86) (end 134.5 119.5) (width 0.2) (layer "F.Cu") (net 9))
 (segment (start 134.5 113.76) (end 134.5 119.5) (width 0.2) (layer "F.Cu") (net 9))
 (segment (start 180.23 117.86) (end 136.14 117.86) (width 0.2) (layer "F.Cu") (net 9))
 (segment (start 123.5 102.76) (end 134.5 113.76) (width 0.2) (layer "F.Cu") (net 9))
 (segment (start 115.88 97.68) (end 118.42 97.68) (width 0.2) (layer "B.Cu") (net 9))
 (segment (start 118.42 97.68) (end 123.5 102.76) (width 0.2) (layer "B.Cu") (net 9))
 (segment (start 116.98 91.5) (end 115.88 92.6) (width 0.2) (layer "F.Cu") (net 19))
 (segment (start 128.42 74) (end 116.98 85.44) (width 0.2) (layer "F.Cu") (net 19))
 (segment (start 116.98 85.44) (end 116.98 91.5) (width 0.2) (layer "F.Cu") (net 19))
 (segment (start 131.44 84.98) (end 123.5 84.98) (width 0.2) (layer "B.Cu") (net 15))
 (segment (start 142.42 74) (end 131.44 84.98) (width 0.2) (layer "B.Cu") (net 15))
 (segment (start 124.9 92.6) (end 123.5 92.6) (width 0.2) (layer "B.Cu") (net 12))
 (segment (start 142.4 75.1) (end 124.9 92.6) (width 0.2) (layer "B.Cu") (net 12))
 (segment (start 154.82 75.1) (end 142.4 75.1) (width 0.2) (layer "B.Cu") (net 12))
 (segment (start 155.92 74) (end 154.82 75.1) (width 0.2) (layer "B.Cu") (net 12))
 (segment (start 141.73 110.38) (end 123.5 110.38) (width 0.2) (layer "B.Cu") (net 6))
 (segment (start 165.44 86.67) (end 141.73 110.38) (width 0.2) (layer "B.Cu") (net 6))
 (segment (start 165.44 77.9) (end 165.44 86.67) (width 0.2) (layer "B.Cu") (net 6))
 (segment (start 169.34 74) (end 165.44 77.9) (width 0.2) (layer "B.Cu") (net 6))
 (segment (start 181.5 117.86) (end 181.5 116.91) (width 0.2) (layer "B.Cu") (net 22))
 (segment (start 181.4 116.81) (end 153.295585 116.81) (width 0.2) (layer "B.Cu") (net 22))
 (segment (start 153.295585 116.81) (end 133.605585 136.5) (width 0.2) (layer "B.Cu") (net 22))
 (segment (start 114.78 127.385585) (end 114.78 106.4) (width 0.2) (layer "B.Cu") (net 22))
 (segment (start 133.605585 136.5) (end 123.894415 136.5) (width 0.2) (layer "B.Cu") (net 22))
 (segment (start 114.78 106.4) (end 115.88 105.3) (width 0.2) (layer "B.Cu") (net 22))
 (segment (start 181.5 116.91) (end 181.4 116.81) (width 0.2) (layer "B.Cu") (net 22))
 (segment (start 123.894415 136.5) (end 114.78 127.385585) (width 0.2) (layer "B.Cu") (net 22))
 (segment (start 128.214214 135.5) (end 127.5 135.5) (width 0.2) (layer "F.Cu") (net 30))
 (segment (start 133.53 130.184214) (end 128.214214 135.5) (width 0.2) (layer "F.Cu") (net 30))
 (segment (start 133.53 119.5) (end 133.53 130.184214) (width 0.2) (layer "F.Cu") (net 30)))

